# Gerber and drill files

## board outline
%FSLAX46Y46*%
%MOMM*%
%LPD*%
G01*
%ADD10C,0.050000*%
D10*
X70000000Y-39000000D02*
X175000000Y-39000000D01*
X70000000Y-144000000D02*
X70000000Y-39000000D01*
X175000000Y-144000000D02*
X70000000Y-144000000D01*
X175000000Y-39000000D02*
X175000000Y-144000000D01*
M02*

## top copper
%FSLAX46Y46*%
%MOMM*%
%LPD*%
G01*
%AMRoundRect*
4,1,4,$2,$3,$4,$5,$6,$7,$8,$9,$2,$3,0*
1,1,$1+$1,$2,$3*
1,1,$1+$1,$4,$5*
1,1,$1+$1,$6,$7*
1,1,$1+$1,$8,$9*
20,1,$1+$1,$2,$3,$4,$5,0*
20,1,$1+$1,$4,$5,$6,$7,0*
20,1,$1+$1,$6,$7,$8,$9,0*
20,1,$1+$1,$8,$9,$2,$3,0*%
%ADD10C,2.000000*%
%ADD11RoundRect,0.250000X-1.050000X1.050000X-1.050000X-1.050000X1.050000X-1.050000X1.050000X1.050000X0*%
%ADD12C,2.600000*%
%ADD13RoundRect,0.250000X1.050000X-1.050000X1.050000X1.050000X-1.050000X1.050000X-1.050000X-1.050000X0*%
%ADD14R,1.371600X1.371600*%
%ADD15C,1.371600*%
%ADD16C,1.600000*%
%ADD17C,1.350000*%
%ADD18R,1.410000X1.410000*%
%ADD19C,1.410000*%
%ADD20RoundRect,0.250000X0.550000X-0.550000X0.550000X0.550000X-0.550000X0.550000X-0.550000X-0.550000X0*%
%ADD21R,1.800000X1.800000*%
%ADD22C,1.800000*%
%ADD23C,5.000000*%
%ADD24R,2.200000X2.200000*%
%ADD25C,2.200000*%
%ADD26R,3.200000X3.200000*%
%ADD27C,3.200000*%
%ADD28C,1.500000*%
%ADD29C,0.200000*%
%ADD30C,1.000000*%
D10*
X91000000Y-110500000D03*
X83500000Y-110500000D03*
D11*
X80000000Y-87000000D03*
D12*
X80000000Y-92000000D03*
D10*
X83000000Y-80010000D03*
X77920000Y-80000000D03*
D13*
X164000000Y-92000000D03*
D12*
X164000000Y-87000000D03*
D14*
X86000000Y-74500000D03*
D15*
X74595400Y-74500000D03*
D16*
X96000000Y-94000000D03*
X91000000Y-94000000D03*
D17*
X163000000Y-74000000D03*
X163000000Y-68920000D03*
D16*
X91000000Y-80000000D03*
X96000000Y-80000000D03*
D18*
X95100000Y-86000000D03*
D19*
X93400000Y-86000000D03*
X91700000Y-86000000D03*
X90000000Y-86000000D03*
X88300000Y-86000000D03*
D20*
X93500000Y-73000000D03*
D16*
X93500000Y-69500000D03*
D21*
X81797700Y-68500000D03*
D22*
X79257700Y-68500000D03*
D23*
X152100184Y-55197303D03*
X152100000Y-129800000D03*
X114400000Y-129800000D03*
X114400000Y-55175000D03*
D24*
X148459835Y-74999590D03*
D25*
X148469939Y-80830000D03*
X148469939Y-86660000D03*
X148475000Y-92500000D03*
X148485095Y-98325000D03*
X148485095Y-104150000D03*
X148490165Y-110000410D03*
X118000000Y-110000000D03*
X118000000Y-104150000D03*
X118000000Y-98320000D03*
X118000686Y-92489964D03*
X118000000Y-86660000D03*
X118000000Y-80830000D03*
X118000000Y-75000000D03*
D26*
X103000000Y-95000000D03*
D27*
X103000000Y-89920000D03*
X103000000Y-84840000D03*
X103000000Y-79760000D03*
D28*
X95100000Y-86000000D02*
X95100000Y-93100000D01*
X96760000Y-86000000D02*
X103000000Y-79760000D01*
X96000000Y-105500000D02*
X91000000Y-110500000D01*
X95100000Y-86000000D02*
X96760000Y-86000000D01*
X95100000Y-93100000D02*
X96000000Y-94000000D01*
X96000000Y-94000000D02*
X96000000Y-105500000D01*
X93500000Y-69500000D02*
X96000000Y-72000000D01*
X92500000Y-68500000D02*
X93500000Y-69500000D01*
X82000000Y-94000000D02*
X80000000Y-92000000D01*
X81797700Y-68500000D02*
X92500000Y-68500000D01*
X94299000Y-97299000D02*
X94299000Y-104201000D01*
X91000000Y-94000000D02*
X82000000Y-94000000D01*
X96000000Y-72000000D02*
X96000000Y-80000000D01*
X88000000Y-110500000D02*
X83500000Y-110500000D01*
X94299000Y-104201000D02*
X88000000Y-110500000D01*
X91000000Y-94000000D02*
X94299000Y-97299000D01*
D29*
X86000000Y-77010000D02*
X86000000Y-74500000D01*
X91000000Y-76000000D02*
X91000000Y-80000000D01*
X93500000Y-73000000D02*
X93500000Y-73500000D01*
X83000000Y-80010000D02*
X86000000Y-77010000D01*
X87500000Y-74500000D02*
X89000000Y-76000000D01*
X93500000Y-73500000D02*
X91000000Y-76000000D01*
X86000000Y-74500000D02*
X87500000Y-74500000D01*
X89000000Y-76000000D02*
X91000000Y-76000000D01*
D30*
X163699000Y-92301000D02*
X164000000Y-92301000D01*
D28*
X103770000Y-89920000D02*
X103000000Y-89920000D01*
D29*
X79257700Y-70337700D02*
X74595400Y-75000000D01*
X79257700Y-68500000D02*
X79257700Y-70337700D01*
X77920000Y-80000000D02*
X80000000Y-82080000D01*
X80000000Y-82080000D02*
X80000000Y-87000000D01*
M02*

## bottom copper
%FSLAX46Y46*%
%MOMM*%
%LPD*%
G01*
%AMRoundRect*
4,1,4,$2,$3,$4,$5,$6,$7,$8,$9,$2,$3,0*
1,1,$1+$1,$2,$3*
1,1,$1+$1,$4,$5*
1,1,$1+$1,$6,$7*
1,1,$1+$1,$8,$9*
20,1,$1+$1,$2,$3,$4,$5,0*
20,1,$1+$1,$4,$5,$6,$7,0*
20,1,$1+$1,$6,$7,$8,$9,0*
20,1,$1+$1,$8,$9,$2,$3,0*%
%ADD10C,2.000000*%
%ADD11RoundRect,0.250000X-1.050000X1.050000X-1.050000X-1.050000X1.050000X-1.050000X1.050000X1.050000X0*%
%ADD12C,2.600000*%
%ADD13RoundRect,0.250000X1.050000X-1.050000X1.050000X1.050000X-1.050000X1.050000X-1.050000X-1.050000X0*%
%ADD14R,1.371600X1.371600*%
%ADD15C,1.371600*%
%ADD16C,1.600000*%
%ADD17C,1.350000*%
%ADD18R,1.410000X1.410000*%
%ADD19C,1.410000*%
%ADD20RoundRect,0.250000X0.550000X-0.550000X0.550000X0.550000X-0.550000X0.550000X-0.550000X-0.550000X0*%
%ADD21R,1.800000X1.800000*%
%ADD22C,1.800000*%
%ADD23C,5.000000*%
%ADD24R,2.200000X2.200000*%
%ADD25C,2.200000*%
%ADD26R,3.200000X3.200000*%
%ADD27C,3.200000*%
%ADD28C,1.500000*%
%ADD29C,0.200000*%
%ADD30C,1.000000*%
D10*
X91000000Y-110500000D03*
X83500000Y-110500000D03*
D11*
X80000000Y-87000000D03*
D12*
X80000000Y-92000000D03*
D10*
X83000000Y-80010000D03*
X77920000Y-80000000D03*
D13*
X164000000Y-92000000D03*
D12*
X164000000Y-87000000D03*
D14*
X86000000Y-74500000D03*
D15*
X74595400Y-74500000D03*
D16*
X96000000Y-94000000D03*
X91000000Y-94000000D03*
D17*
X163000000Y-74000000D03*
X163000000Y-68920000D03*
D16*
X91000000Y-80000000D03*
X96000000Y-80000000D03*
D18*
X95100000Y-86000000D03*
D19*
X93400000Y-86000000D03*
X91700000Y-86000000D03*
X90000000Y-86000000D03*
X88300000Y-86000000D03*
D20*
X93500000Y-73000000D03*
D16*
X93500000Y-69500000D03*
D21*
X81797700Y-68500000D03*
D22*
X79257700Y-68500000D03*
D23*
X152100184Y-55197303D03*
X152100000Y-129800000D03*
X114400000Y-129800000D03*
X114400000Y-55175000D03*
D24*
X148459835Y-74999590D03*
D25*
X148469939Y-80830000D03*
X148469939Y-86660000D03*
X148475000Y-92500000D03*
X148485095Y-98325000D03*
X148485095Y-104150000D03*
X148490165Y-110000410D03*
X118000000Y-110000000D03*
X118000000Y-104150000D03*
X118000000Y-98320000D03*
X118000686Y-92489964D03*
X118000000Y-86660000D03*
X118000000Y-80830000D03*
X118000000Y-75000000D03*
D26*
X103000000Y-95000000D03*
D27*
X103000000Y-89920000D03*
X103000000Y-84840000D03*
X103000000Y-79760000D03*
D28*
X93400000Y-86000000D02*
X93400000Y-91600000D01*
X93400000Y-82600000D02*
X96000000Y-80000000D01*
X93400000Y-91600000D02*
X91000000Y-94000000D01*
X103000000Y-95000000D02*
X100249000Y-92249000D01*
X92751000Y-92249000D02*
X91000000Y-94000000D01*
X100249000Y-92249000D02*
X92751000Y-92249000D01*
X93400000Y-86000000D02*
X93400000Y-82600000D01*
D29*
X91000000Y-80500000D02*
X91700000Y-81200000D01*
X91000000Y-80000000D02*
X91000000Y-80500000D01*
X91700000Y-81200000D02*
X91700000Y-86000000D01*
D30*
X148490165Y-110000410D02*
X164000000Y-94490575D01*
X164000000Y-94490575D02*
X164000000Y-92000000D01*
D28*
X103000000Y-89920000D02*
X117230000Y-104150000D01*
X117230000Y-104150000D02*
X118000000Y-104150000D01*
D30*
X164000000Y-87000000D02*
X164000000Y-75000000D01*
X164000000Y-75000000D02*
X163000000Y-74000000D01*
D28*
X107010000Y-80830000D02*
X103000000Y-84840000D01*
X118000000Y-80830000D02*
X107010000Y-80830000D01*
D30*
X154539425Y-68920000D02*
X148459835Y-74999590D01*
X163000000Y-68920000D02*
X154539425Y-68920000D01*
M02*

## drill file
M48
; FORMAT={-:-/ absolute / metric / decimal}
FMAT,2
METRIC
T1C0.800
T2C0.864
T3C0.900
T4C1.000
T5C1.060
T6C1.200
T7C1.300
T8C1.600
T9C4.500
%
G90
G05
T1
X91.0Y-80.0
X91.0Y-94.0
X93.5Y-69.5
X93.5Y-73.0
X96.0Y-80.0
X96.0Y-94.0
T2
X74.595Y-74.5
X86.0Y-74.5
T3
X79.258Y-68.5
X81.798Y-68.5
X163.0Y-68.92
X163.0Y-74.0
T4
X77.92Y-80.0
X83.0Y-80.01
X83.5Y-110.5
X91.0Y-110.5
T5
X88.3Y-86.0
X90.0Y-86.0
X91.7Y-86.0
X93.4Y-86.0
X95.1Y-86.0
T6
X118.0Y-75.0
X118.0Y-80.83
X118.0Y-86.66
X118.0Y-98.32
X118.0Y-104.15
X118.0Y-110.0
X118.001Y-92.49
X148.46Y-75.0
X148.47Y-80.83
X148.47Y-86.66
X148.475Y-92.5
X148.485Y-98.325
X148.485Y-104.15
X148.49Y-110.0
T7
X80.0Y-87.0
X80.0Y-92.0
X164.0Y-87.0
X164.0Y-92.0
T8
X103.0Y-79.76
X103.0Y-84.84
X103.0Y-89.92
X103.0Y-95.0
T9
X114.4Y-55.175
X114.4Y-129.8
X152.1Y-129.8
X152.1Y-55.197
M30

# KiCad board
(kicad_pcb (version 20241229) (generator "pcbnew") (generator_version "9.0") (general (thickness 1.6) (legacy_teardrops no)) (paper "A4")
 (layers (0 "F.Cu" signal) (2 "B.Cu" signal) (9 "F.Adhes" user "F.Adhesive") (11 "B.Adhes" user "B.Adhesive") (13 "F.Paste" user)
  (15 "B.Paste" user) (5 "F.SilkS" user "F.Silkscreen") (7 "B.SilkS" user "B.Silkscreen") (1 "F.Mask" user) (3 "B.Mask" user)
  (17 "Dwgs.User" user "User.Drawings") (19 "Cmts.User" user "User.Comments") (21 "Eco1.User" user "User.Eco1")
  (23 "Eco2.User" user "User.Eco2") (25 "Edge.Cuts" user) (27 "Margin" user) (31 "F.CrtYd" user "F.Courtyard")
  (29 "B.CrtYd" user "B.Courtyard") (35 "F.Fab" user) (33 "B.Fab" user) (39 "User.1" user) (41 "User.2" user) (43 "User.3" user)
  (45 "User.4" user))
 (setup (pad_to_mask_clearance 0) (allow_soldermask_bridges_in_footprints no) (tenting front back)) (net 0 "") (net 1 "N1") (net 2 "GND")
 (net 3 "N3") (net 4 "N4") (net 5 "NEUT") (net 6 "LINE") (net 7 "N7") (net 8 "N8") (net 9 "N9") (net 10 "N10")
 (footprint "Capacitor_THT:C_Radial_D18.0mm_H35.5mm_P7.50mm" (layer "F.Cu") (at 91 110.5 180)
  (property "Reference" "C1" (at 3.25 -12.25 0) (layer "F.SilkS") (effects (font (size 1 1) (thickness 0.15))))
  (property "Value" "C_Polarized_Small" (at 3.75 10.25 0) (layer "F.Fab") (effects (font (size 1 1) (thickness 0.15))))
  (pad "1" thru_hole circle (at 0 0 180) (size 2 2) (drill 1) (layers "*.Cu" "*.Mask") (remove_unused_layers no) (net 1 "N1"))
  (pad "2" thru_hole circle (at 7.5 0 180) (size 2 2) (drill 1) (layers "*.Cu" "*.Mask") (remove_unused_layers no) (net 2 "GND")))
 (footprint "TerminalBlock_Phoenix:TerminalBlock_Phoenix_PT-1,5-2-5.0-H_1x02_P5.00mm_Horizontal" (layer "F.Cu") (at 80 87 -90)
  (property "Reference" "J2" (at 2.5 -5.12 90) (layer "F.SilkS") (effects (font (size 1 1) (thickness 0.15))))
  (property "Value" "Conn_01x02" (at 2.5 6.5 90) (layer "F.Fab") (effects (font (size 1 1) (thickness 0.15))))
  (pad "1" thru_hole roundrect (at 0 0 270) (size 2.6 2.6) (drill 1.3) (layers "*.Cu" "*.Mask") (remove_unused_layers no)
   (roundrect_rratio 0.096154) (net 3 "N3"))
  (pad "2" thru_hole circle (at 5 0 270) (size 2.6 2.6) (drill 1.3) (layers "*.Cu" "*.Mask") (remove_unused_layers no) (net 2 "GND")))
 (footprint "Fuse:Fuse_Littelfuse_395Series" (layer "F.Cu") (at 83 80.01 180)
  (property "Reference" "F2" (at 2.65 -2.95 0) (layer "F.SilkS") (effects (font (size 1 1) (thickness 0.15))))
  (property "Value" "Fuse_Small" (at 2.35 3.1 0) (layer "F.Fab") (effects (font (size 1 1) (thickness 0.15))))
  (pad "1" thru_hole circle (at 0 0 180) (size 2 2) (drill 1) (layers "*.Cu" "*.Mask") (remove_unused_layers no) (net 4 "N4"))
  (pad "2" thru_hole circle (at 5.08 0.01 180) (size 2 2) (drill 1) (layers "*.Cu" "*.Mask") (remove_unused_layers no) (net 3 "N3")))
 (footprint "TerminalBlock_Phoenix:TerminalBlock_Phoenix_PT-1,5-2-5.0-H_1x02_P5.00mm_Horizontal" (layer "F.Cu") (at 164 92 90)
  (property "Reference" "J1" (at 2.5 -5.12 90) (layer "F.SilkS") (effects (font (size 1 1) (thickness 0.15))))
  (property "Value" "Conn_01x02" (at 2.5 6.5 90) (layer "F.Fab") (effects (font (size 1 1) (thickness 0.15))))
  (pad "1" thru_hole roundrect (at 0 0 90) (size 2.6 2.6) (drill 1.3) (layers "*.Cu" "*.Mask") (remove_unused_layers no)
   (roundrect_rratio 0.096154) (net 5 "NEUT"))
  (pad "2" thru_hole circle (at 5 0 90) (size 2.6 2.6) (drill 1.3) (layers "*.Cu" "*.Mask") (remove_unused_layers no) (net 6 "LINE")))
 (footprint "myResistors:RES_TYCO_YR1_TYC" (layer "F.Cu") (at 86 74.5 180)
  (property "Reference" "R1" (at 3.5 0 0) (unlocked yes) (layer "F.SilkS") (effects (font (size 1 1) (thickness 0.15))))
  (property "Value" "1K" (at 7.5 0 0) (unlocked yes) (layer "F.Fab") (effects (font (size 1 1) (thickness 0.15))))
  (pad "1" thru_hole rect (at 0 0 180) (size 1.3716 1.3716) (drill 0.8636) (layers "*.Cu" "*.Mask") (remove_unused_layers no) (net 4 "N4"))
  (pad "2" thru_hole circle (at 11.4046 0 180) (size 1.3716 1.3716) (drill 0.8636) (layers "*.Cu" "*.Mask") (remove_unused_layers no)
   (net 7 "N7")))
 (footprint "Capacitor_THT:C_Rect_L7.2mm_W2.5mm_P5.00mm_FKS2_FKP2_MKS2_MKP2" (layer "F.Cu") (at 96 94 180)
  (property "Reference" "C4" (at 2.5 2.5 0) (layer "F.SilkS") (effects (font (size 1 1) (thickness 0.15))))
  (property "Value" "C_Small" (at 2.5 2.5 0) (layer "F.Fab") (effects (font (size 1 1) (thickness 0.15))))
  (pad "1" thru_hole circle (at 0 0 180) (size 1.6 1.6) (drill 0.8) (layers "*.Cu" "*.Mask") (remove_unused_layers no) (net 1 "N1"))
  (pad "2" thru_hole circle (at 5 0 180) (size 1.6 1.6) (drill 0.8) (layers "*.Cu" "*.Mask") (remove_unused_layers no) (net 2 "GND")))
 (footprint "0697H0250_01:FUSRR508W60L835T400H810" (layer "F.Cu") (at 163 71.46 90)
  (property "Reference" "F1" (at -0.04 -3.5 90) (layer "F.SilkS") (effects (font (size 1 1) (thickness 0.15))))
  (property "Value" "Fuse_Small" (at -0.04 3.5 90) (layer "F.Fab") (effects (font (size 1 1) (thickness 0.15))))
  (pad "1" thru_hole circle (at -2.54 0 90) (size 1.35 1.35) (drill 0.9) (layers "*.Cu" "*.Mask") (remove_unused_layers no) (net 6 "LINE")
   (solder_mask_margin 0.102))
  (pad "2" thru_hole circle (at 2.54 0 90) (size 1.35 1.35) (drill 0.9) (layers "*.Cu" "*.Mask") (remove_unused_layers no) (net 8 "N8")
   (solder_mask_margin 0.102)))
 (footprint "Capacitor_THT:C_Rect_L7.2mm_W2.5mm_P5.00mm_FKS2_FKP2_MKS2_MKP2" (layer "F.Cu") (at 91 80)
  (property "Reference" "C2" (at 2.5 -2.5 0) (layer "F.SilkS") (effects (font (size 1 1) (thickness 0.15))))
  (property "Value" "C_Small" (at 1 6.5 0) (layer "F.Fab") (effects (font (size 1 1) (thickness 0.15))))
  (pad "1" thru_hole circle (at 0 0) (size 1.6 1.6) (drill 0.8) (layers "*.Cu" "*.Mask") (remove_unused_layers no) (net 4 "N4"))
  (pad "2" thru_hole circle (at 5 0) (size 1.6 1.6) (drill 0.8) (layers "*.Cu" "*.Mask") (remove_unused_layers no) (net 2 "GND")))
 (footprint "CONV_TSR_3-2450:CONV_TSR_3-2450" (layer "F.Cu") (at 91.7 86)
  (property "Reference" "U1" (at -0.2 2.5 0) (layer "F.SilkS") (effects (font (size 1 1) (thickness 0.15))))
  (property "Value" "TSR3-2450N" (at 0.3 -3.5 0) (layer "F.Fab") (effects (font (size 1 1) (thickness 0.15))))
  (pad "1" thru_hole rect (at 3.4 0) (size 1.41 1.41) (drill 1.06) (layers "*.Cu" "*.Mask") (remove_unused_layers no) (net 1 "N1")
   (solder_mask_margin 0.102))
  (pad "2" thru_hole circle (at 1.7 0) (size 1.41 1.41) (drill 1.06) (layers "*.Cu" "*.Mask") (remove_unused_layers no) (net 2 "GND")
   (solder_mask_margin 0.102))
  (pad "3" thru_hole circle (at 0 0) (size 1.41 1.41) (drill 1.06) (layers "*.Cu" "*.Mask") (remove_unused_layers no) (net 4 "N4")
   (solder_mask_margin 0.102))
  (pad "4" thru_hole circle (at -1.7 0) (size 1.41 1.41) (drill 1.06) (layers "*.Cu" "*.Mask") (remove_unused_layers no)
   (solder_mask_margin 0.102))
  (pad "5" thru_hole circle (at -3.4 0) (size 1.41 1.41) (drill 1.06) (layers "*.Cu" "*.Mask") (remove_unused_layers no)
   (solder_mask_margin 0.102)))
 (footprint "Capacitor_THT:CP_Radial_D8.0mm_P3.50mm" (layer "F.Cu") (at 93.5 73 90)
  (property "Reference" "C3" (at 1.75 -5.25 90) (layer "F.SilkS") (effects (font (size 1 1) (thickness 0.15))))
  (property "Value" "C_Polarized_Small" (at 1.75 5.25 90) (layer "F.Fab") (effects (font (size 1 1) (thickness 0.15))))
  (pad "1" thru_hole roundrect (at 0 0 90) (size 1.6 1.6) (drill 0.8) (layers "*.Cu" "*.Mask") (remove_unused_layers no)
   (roundrect_rratio 0.15625) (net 4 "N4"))
  (pad "2" thru_hole circle (at 3.5 0 90) (size 1.6 1.6) (drill 0.8) (layers "*.Cu" "*.Mask") (remove_unused_layers no) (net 2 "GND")))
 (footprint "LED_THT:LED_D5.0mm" (layer "F.Cu") (at 81.7977 68.5 180)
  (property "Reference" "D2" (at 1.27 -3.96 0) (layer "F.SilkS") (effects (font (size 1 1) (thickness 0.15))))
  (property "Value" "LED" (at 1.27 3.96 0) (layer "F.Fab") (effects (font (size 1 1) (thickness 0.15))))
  (pad "1" thru_hole rect (at 0 0 180) (size 1.8 1.8) (drill 0.9) (layers "*.Cu" "*.Mask") (remove_unused_layers no) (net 2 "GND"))
  (pad "2" thru_hole circle (at 2.54 0 180) (size 1.8 1.8) (drill 0.9) (layers "*.Cu" "*.Mask") (remove_unused_layers no) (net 7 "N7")))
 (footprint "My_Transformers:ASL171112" (layer "F.Cu") (at 133.35 81.45 180)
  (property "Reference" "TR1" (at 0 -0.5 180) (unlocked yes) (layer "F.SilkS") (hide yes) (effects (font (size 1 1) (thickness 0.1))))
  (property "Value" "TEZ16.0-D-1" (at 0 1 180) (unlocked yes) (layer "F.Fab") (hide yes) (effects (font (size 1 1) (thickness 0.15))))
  (pad "" np_thru_hole circle (at -18.750184 26.252697 180) (size 5 5) (drill 4.5) (layers "*.Cu" "*.Mask"))
  (pad "" np_thru_hole circle (at -18.75 -48.35 180) (size 5 5) (drill 4.5) (layers "*.Cu" "*.Mask"))
  (pad "" np_thru_hole circle (at 18.95 -48.35 180) (size 5 5) (drill 4.5) (layers "*.Cu" "*.Mask"))
  (pad "" np_thru_hole circle (at 18.95 26.275 180) (size 5 5) (drill 4.5) (layers "*.Cu" "*.Mask"))
  (pad "1" thru_hole rect (at -15.109835 6.45041 180) (size 2.2 2.2) (drill 1.2) (layers "*.Cu" "*.Mask") (remove_unused_layers no)
   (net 8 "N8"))
  (pad "2" thru_hole circle (at -15.119939 0.62 180) (size 2.2 2.2) (drill 1.2) (layers "*.Cu" "*.Mask") (remove_unused_layers no))
  (pad "3" thru_hole circle (at -15.119939 -5.21 180) (size 2.2 2.2) (drill 1.2) (layers "*.Cu" "*.Mask") (remove_unused_layers no))
  (pad "4" thru_hole circle (at -15.125 -11.05 180) (size 2.2 2.2) (drill 1.2) (layers "*.Cu" "*.Mask") (remove_unused_layers no))
  (pad "5" thru_hole circle (at -15.135095 -16.875 180) (size 2.2 2.2) (drill 1.2) (layers "*.Cu" "*.Mask") (remove_unused_layers no))
  (pad "6" thru_hole circle (at -15.135095 -22.7 180) (size 2.2 2.2) (drill 1.2) (layers "*.Cu" "*.Mask") (remove_unused_layers no))
  (pad "7" thru_hole circle (at -15.140165 -28.55041 180) (size 2.2 2.2) (drill 1.2) (layers "*.Cu" "*.Mask") (remove_unused_layers no)
   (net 5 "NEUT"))
  (pad "8" thru_hole circle (at 15.35 -28.55 180) (size 2.2 2.2) (drill 1.2) (layers "*.Cu" "*.Mask") (remove_unused_layers no))
  (pad "9" thru_hole circle (at 15.35 -22.7 180) (size 2.2 2.2) (drill 1.2) (layers "*.Cu" "*.Mask") (remove_unused_layers no) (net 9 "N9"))
  (pad "10" thru_hole circle (at 15.35 -16.87 180) (size 2.2 2.2) (drill 1.2) (layers "*.Cu" "*.Mask") (remove_unused_layers no))
  (pad "11" thru_hole circle (at 15.349314 -11.039964 180) (size 2.2 2.2) (drill 1.2) (layers "*.Cu" "*.Mask") (remove_unused_layers no))
  (pad "12" thru_hole circle (at 15.35 -5.21 180) (size 2.2 2.2) (drill 1.2) (layers "*.Cu" "*.Mask") (remove_unused_layers no))
  (pad "13" thru_hole circle (at 15.35 0.62 180) (size 2.2 2.2) (drill 1.2) (layers "*.Cu" "*.Mask") (remove_unused_layers no)
   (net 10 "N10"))
  (pad "14" thru_hole circle (at 15.35 6.45 180) (size 2.2 2.2) (drill 1.2) (layers "*.Cu" "*.Mask") (remove_unused_layers no)))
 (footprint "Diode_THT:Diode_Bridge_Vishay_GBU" (layer "F.Cu") (at 103 95 90)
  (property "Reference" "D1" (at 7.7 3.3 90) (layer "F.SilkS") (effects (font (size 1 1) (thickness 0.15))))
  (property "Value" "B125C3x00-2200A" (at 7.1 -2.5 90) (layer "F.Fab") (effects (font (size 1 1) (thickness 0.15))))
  (pad "1" thru_hole rect (at 0 0 90) (size 3.2 3.2) (drill 1.6) (layers "*.Cu" "*.Mask") (remove_unused_layers no) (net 2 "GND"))
  (pad "2" thru_hole circle (at 5.08 0 90) (size 3.2 3.2) (drill 1.6) (layers "*.Cu" "*.Mask") (remove_unused_layers no) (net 9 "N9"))
  (pad "3" thru_hole circle (at 10.16 0 90) (size 3.2 3.2) (drill 1.6) (layers "*.Cu" "*.Mask") (remove_unused_layers no) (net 10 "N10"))
  (pad "4" thru_hole circle (at 15.24 0 90) (size 3.2 3.2) (drill 1.6) (layers "*.Cu" "*.Mask") (remove_unused_layers no) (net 1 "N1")))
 (gr_line (start 70 39) (end 175 39) (stroke (width 0.05) (type default)) (layer "Edge.Cuts"))
 (gr_line (start 70 144) (end 70 39) (stroke (width 0.05) (type default)) (layer "Edge.Cuts"))
 (gr_line (start 175 144) (end 70 144) (stroke (width 0.05) (type default)) (layer "Edge.Cuts"))
 (gr_line (start 175 39) (end 175 144) (stroke (width 0.05) (type default)) (layer "Edge.Cuts"))
 (segment (start 95.1 86) (end 95.1 93.1) (width 1.5) (layer "F.Cu") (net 1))
 (segment (start 96.76 86) (end 103 79.76) (width 1.5) (layer "F.Cu") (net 1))
 (segment (start 96 105.5) (end 91 110.5) (width 1.5) (layer "F.Cu") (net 1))
 (segment (start 95.1 86) (end 96.76 86) (width 1.5) (layer "F.Cu") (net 1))
 (segment (start 95.1 93.1) (end 96 94) (width 1.5) (layer "F.Cu") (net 1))
 (segment (start 96 94) (end 96 105.5) (width 1.5) (layer "F.Cu") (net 1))
 (segment (start 93.5 69.5) (end 96 72) (width 1.5) (layer "F.Cu") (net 2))
 (segment (start 92.5 68.5) (end 93.5 69.5) (width 1.5) (layer "F.Cu") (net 2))
 (segment (start 82 94) (end 80 92) (width 1.5) (layer "F.Cu") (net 2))
 (segment (start 81.7977 68.5) (end 92.5 68.5) (width 1.5) (layer "F.Cu") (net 2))
 (segment (start 94.299 97.299) (end 94.299 104.201) (width 1.5) (layer "F.Cu") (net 2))
 (segment (start 91 94) (end 82 94) (width 1.5) (layer "F.Cu") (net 2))
 (segment (start 96 72) (end 96 80) (width 1.5) (layer "F.Cu") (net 2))
 (segment (start 88 110.5) (end 83.5 110.5) (width 1.5) (layer "F.Cu") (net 2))
 (segment (start 94.299 104.201) (end 88 110.5) (width 1.5) (layer "F.Cu") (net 2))
 (segment (start 91 94) (end 94.299 97.299) (width 1.5) (layer "F.Cu") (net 2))
 (segment (start 93.4 86) (end 93.4 91.6) (width 1.5) (layer "B.Cu") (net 2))
 (segment (start 93.4 82.6) (end 96 80) (width 1.5) (layer "B.Cu") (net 2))
 (segment (start 93.4 91.6) (end 91 94) (width 1.5) (layer "B.Cu") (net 2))
 (segment (start 103 95) (end 100.249 92.249) (width 1.5) (layer "B.Cu") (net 2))
 (segment (start 92.751 92.249) (end 91 94) (width 1.5) (layer "B.Cu") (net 2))
 (segment (start 100.249 92.249) (end 92.751 92.249) (width 1.5) (layer "B.Cu") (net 2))
 (segment (start 93.4 86) (end 93.4 82.6) (width 1.5) (layer "B.Cu") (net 2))
 (segment (start 86 77.01) (end 86 74.5) (width 0.2) (layer "F.Cu") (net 4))
 (segment (start 91 76) (end 91 80) (width 0.2) (layer "F.Cu") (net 4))
 (segment (start 93.5 73) (end 93.5 73.5) (width 0.2) (layer "F.Cu") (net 4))
 (segment (start 83 80.01) (end 86 77.01) (width 0.2) (layer "F.Cu") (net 4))
 (segment (start 87.5 74.5) (end 89 76) (width 0.2) (layer "F.Cu") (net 4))
 (segment (start 93.5 73.5) (end 91 76) (width 0.2) (layer "F.Cu") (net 4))
 (segment (start 86 74.5) (end 87.5 74.5) (width 0.2) (layer "F.Cu") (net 4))
 (segment (start 89 76) (end 91 76) (width 0.2) (layer "F.Cu") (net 4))
 (segment (start 91 80.5) (end 91.7 81.2) (width 0.2) (layer "B.Cu") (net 4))
 (segment (start 91 80) (end 91 80.5) (width 0.2) (layer "B.Cu") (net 4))
 (segment (start 91.7 81.2) (end 91.7 86) (width 0.2) (layer "B.Cu") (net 4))
 (segment (start 163.699 92.301) (end 164 92.301) (width 1) (layer "F.Cu") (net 5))
 (segment (start 148.490165 110.00041) (end 164 94.490575) (width 1) (layer "B.Cu") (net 5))
 (segment (start 164 94.490575) (end 164 92) (width 1) (layer "B.Cu") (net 5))
 (segment (start 103.77 89.92) (end 103 89.92) (width 1.5) (layer "F.Cu") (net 9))
 (segment (start 103 89.92) (end 117.23 104.15) (width 1.5) (layer "B.Cu") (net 9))
 (segment (start 117.23 104.15) (end 118 104.15) (width 1.5) (layer "B.Cu") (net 9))
 (segment (start 79.2577 70.3377) (end 74.5954 75) (width 0.2) (layer "F.Cu") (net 7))
 (segment (start 79.2577 68.5) (end 79.2577 70.3377) (width 0.2) (layer "F.Cu") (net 7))
 (segment (start 164 87) (end 164 75) (width 1) (layer "B.Cu") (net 6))
 (segment (start 164 75) (end 163 74) (width 1) (layer "B.Cu") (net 6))
 (segment (start 77.92 80) (end 80 82.08) (width 0.2) (layer "F.Cu") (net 3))
 (segment (start 80 82.08) (end 80 87) (width 0.2) (layer "F.Cu") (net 3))
 (segment (start 107.01 80.83) (end 103 84.84) (width 1.5) (layer "B.Cu") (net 10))
 (segment (start 118 80.83) (end 107.01 80.83) (width 1.5) (layer "B.Cu") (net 10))
 (segment (start 154.539425 68.92) (end 148.459835 74.99959) (width 1) (layer "B.Cu") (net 8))
 (segment (start 163 68.92) (end 154.539425 68.92) (width 1) (layer "B.Cu") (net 8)))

